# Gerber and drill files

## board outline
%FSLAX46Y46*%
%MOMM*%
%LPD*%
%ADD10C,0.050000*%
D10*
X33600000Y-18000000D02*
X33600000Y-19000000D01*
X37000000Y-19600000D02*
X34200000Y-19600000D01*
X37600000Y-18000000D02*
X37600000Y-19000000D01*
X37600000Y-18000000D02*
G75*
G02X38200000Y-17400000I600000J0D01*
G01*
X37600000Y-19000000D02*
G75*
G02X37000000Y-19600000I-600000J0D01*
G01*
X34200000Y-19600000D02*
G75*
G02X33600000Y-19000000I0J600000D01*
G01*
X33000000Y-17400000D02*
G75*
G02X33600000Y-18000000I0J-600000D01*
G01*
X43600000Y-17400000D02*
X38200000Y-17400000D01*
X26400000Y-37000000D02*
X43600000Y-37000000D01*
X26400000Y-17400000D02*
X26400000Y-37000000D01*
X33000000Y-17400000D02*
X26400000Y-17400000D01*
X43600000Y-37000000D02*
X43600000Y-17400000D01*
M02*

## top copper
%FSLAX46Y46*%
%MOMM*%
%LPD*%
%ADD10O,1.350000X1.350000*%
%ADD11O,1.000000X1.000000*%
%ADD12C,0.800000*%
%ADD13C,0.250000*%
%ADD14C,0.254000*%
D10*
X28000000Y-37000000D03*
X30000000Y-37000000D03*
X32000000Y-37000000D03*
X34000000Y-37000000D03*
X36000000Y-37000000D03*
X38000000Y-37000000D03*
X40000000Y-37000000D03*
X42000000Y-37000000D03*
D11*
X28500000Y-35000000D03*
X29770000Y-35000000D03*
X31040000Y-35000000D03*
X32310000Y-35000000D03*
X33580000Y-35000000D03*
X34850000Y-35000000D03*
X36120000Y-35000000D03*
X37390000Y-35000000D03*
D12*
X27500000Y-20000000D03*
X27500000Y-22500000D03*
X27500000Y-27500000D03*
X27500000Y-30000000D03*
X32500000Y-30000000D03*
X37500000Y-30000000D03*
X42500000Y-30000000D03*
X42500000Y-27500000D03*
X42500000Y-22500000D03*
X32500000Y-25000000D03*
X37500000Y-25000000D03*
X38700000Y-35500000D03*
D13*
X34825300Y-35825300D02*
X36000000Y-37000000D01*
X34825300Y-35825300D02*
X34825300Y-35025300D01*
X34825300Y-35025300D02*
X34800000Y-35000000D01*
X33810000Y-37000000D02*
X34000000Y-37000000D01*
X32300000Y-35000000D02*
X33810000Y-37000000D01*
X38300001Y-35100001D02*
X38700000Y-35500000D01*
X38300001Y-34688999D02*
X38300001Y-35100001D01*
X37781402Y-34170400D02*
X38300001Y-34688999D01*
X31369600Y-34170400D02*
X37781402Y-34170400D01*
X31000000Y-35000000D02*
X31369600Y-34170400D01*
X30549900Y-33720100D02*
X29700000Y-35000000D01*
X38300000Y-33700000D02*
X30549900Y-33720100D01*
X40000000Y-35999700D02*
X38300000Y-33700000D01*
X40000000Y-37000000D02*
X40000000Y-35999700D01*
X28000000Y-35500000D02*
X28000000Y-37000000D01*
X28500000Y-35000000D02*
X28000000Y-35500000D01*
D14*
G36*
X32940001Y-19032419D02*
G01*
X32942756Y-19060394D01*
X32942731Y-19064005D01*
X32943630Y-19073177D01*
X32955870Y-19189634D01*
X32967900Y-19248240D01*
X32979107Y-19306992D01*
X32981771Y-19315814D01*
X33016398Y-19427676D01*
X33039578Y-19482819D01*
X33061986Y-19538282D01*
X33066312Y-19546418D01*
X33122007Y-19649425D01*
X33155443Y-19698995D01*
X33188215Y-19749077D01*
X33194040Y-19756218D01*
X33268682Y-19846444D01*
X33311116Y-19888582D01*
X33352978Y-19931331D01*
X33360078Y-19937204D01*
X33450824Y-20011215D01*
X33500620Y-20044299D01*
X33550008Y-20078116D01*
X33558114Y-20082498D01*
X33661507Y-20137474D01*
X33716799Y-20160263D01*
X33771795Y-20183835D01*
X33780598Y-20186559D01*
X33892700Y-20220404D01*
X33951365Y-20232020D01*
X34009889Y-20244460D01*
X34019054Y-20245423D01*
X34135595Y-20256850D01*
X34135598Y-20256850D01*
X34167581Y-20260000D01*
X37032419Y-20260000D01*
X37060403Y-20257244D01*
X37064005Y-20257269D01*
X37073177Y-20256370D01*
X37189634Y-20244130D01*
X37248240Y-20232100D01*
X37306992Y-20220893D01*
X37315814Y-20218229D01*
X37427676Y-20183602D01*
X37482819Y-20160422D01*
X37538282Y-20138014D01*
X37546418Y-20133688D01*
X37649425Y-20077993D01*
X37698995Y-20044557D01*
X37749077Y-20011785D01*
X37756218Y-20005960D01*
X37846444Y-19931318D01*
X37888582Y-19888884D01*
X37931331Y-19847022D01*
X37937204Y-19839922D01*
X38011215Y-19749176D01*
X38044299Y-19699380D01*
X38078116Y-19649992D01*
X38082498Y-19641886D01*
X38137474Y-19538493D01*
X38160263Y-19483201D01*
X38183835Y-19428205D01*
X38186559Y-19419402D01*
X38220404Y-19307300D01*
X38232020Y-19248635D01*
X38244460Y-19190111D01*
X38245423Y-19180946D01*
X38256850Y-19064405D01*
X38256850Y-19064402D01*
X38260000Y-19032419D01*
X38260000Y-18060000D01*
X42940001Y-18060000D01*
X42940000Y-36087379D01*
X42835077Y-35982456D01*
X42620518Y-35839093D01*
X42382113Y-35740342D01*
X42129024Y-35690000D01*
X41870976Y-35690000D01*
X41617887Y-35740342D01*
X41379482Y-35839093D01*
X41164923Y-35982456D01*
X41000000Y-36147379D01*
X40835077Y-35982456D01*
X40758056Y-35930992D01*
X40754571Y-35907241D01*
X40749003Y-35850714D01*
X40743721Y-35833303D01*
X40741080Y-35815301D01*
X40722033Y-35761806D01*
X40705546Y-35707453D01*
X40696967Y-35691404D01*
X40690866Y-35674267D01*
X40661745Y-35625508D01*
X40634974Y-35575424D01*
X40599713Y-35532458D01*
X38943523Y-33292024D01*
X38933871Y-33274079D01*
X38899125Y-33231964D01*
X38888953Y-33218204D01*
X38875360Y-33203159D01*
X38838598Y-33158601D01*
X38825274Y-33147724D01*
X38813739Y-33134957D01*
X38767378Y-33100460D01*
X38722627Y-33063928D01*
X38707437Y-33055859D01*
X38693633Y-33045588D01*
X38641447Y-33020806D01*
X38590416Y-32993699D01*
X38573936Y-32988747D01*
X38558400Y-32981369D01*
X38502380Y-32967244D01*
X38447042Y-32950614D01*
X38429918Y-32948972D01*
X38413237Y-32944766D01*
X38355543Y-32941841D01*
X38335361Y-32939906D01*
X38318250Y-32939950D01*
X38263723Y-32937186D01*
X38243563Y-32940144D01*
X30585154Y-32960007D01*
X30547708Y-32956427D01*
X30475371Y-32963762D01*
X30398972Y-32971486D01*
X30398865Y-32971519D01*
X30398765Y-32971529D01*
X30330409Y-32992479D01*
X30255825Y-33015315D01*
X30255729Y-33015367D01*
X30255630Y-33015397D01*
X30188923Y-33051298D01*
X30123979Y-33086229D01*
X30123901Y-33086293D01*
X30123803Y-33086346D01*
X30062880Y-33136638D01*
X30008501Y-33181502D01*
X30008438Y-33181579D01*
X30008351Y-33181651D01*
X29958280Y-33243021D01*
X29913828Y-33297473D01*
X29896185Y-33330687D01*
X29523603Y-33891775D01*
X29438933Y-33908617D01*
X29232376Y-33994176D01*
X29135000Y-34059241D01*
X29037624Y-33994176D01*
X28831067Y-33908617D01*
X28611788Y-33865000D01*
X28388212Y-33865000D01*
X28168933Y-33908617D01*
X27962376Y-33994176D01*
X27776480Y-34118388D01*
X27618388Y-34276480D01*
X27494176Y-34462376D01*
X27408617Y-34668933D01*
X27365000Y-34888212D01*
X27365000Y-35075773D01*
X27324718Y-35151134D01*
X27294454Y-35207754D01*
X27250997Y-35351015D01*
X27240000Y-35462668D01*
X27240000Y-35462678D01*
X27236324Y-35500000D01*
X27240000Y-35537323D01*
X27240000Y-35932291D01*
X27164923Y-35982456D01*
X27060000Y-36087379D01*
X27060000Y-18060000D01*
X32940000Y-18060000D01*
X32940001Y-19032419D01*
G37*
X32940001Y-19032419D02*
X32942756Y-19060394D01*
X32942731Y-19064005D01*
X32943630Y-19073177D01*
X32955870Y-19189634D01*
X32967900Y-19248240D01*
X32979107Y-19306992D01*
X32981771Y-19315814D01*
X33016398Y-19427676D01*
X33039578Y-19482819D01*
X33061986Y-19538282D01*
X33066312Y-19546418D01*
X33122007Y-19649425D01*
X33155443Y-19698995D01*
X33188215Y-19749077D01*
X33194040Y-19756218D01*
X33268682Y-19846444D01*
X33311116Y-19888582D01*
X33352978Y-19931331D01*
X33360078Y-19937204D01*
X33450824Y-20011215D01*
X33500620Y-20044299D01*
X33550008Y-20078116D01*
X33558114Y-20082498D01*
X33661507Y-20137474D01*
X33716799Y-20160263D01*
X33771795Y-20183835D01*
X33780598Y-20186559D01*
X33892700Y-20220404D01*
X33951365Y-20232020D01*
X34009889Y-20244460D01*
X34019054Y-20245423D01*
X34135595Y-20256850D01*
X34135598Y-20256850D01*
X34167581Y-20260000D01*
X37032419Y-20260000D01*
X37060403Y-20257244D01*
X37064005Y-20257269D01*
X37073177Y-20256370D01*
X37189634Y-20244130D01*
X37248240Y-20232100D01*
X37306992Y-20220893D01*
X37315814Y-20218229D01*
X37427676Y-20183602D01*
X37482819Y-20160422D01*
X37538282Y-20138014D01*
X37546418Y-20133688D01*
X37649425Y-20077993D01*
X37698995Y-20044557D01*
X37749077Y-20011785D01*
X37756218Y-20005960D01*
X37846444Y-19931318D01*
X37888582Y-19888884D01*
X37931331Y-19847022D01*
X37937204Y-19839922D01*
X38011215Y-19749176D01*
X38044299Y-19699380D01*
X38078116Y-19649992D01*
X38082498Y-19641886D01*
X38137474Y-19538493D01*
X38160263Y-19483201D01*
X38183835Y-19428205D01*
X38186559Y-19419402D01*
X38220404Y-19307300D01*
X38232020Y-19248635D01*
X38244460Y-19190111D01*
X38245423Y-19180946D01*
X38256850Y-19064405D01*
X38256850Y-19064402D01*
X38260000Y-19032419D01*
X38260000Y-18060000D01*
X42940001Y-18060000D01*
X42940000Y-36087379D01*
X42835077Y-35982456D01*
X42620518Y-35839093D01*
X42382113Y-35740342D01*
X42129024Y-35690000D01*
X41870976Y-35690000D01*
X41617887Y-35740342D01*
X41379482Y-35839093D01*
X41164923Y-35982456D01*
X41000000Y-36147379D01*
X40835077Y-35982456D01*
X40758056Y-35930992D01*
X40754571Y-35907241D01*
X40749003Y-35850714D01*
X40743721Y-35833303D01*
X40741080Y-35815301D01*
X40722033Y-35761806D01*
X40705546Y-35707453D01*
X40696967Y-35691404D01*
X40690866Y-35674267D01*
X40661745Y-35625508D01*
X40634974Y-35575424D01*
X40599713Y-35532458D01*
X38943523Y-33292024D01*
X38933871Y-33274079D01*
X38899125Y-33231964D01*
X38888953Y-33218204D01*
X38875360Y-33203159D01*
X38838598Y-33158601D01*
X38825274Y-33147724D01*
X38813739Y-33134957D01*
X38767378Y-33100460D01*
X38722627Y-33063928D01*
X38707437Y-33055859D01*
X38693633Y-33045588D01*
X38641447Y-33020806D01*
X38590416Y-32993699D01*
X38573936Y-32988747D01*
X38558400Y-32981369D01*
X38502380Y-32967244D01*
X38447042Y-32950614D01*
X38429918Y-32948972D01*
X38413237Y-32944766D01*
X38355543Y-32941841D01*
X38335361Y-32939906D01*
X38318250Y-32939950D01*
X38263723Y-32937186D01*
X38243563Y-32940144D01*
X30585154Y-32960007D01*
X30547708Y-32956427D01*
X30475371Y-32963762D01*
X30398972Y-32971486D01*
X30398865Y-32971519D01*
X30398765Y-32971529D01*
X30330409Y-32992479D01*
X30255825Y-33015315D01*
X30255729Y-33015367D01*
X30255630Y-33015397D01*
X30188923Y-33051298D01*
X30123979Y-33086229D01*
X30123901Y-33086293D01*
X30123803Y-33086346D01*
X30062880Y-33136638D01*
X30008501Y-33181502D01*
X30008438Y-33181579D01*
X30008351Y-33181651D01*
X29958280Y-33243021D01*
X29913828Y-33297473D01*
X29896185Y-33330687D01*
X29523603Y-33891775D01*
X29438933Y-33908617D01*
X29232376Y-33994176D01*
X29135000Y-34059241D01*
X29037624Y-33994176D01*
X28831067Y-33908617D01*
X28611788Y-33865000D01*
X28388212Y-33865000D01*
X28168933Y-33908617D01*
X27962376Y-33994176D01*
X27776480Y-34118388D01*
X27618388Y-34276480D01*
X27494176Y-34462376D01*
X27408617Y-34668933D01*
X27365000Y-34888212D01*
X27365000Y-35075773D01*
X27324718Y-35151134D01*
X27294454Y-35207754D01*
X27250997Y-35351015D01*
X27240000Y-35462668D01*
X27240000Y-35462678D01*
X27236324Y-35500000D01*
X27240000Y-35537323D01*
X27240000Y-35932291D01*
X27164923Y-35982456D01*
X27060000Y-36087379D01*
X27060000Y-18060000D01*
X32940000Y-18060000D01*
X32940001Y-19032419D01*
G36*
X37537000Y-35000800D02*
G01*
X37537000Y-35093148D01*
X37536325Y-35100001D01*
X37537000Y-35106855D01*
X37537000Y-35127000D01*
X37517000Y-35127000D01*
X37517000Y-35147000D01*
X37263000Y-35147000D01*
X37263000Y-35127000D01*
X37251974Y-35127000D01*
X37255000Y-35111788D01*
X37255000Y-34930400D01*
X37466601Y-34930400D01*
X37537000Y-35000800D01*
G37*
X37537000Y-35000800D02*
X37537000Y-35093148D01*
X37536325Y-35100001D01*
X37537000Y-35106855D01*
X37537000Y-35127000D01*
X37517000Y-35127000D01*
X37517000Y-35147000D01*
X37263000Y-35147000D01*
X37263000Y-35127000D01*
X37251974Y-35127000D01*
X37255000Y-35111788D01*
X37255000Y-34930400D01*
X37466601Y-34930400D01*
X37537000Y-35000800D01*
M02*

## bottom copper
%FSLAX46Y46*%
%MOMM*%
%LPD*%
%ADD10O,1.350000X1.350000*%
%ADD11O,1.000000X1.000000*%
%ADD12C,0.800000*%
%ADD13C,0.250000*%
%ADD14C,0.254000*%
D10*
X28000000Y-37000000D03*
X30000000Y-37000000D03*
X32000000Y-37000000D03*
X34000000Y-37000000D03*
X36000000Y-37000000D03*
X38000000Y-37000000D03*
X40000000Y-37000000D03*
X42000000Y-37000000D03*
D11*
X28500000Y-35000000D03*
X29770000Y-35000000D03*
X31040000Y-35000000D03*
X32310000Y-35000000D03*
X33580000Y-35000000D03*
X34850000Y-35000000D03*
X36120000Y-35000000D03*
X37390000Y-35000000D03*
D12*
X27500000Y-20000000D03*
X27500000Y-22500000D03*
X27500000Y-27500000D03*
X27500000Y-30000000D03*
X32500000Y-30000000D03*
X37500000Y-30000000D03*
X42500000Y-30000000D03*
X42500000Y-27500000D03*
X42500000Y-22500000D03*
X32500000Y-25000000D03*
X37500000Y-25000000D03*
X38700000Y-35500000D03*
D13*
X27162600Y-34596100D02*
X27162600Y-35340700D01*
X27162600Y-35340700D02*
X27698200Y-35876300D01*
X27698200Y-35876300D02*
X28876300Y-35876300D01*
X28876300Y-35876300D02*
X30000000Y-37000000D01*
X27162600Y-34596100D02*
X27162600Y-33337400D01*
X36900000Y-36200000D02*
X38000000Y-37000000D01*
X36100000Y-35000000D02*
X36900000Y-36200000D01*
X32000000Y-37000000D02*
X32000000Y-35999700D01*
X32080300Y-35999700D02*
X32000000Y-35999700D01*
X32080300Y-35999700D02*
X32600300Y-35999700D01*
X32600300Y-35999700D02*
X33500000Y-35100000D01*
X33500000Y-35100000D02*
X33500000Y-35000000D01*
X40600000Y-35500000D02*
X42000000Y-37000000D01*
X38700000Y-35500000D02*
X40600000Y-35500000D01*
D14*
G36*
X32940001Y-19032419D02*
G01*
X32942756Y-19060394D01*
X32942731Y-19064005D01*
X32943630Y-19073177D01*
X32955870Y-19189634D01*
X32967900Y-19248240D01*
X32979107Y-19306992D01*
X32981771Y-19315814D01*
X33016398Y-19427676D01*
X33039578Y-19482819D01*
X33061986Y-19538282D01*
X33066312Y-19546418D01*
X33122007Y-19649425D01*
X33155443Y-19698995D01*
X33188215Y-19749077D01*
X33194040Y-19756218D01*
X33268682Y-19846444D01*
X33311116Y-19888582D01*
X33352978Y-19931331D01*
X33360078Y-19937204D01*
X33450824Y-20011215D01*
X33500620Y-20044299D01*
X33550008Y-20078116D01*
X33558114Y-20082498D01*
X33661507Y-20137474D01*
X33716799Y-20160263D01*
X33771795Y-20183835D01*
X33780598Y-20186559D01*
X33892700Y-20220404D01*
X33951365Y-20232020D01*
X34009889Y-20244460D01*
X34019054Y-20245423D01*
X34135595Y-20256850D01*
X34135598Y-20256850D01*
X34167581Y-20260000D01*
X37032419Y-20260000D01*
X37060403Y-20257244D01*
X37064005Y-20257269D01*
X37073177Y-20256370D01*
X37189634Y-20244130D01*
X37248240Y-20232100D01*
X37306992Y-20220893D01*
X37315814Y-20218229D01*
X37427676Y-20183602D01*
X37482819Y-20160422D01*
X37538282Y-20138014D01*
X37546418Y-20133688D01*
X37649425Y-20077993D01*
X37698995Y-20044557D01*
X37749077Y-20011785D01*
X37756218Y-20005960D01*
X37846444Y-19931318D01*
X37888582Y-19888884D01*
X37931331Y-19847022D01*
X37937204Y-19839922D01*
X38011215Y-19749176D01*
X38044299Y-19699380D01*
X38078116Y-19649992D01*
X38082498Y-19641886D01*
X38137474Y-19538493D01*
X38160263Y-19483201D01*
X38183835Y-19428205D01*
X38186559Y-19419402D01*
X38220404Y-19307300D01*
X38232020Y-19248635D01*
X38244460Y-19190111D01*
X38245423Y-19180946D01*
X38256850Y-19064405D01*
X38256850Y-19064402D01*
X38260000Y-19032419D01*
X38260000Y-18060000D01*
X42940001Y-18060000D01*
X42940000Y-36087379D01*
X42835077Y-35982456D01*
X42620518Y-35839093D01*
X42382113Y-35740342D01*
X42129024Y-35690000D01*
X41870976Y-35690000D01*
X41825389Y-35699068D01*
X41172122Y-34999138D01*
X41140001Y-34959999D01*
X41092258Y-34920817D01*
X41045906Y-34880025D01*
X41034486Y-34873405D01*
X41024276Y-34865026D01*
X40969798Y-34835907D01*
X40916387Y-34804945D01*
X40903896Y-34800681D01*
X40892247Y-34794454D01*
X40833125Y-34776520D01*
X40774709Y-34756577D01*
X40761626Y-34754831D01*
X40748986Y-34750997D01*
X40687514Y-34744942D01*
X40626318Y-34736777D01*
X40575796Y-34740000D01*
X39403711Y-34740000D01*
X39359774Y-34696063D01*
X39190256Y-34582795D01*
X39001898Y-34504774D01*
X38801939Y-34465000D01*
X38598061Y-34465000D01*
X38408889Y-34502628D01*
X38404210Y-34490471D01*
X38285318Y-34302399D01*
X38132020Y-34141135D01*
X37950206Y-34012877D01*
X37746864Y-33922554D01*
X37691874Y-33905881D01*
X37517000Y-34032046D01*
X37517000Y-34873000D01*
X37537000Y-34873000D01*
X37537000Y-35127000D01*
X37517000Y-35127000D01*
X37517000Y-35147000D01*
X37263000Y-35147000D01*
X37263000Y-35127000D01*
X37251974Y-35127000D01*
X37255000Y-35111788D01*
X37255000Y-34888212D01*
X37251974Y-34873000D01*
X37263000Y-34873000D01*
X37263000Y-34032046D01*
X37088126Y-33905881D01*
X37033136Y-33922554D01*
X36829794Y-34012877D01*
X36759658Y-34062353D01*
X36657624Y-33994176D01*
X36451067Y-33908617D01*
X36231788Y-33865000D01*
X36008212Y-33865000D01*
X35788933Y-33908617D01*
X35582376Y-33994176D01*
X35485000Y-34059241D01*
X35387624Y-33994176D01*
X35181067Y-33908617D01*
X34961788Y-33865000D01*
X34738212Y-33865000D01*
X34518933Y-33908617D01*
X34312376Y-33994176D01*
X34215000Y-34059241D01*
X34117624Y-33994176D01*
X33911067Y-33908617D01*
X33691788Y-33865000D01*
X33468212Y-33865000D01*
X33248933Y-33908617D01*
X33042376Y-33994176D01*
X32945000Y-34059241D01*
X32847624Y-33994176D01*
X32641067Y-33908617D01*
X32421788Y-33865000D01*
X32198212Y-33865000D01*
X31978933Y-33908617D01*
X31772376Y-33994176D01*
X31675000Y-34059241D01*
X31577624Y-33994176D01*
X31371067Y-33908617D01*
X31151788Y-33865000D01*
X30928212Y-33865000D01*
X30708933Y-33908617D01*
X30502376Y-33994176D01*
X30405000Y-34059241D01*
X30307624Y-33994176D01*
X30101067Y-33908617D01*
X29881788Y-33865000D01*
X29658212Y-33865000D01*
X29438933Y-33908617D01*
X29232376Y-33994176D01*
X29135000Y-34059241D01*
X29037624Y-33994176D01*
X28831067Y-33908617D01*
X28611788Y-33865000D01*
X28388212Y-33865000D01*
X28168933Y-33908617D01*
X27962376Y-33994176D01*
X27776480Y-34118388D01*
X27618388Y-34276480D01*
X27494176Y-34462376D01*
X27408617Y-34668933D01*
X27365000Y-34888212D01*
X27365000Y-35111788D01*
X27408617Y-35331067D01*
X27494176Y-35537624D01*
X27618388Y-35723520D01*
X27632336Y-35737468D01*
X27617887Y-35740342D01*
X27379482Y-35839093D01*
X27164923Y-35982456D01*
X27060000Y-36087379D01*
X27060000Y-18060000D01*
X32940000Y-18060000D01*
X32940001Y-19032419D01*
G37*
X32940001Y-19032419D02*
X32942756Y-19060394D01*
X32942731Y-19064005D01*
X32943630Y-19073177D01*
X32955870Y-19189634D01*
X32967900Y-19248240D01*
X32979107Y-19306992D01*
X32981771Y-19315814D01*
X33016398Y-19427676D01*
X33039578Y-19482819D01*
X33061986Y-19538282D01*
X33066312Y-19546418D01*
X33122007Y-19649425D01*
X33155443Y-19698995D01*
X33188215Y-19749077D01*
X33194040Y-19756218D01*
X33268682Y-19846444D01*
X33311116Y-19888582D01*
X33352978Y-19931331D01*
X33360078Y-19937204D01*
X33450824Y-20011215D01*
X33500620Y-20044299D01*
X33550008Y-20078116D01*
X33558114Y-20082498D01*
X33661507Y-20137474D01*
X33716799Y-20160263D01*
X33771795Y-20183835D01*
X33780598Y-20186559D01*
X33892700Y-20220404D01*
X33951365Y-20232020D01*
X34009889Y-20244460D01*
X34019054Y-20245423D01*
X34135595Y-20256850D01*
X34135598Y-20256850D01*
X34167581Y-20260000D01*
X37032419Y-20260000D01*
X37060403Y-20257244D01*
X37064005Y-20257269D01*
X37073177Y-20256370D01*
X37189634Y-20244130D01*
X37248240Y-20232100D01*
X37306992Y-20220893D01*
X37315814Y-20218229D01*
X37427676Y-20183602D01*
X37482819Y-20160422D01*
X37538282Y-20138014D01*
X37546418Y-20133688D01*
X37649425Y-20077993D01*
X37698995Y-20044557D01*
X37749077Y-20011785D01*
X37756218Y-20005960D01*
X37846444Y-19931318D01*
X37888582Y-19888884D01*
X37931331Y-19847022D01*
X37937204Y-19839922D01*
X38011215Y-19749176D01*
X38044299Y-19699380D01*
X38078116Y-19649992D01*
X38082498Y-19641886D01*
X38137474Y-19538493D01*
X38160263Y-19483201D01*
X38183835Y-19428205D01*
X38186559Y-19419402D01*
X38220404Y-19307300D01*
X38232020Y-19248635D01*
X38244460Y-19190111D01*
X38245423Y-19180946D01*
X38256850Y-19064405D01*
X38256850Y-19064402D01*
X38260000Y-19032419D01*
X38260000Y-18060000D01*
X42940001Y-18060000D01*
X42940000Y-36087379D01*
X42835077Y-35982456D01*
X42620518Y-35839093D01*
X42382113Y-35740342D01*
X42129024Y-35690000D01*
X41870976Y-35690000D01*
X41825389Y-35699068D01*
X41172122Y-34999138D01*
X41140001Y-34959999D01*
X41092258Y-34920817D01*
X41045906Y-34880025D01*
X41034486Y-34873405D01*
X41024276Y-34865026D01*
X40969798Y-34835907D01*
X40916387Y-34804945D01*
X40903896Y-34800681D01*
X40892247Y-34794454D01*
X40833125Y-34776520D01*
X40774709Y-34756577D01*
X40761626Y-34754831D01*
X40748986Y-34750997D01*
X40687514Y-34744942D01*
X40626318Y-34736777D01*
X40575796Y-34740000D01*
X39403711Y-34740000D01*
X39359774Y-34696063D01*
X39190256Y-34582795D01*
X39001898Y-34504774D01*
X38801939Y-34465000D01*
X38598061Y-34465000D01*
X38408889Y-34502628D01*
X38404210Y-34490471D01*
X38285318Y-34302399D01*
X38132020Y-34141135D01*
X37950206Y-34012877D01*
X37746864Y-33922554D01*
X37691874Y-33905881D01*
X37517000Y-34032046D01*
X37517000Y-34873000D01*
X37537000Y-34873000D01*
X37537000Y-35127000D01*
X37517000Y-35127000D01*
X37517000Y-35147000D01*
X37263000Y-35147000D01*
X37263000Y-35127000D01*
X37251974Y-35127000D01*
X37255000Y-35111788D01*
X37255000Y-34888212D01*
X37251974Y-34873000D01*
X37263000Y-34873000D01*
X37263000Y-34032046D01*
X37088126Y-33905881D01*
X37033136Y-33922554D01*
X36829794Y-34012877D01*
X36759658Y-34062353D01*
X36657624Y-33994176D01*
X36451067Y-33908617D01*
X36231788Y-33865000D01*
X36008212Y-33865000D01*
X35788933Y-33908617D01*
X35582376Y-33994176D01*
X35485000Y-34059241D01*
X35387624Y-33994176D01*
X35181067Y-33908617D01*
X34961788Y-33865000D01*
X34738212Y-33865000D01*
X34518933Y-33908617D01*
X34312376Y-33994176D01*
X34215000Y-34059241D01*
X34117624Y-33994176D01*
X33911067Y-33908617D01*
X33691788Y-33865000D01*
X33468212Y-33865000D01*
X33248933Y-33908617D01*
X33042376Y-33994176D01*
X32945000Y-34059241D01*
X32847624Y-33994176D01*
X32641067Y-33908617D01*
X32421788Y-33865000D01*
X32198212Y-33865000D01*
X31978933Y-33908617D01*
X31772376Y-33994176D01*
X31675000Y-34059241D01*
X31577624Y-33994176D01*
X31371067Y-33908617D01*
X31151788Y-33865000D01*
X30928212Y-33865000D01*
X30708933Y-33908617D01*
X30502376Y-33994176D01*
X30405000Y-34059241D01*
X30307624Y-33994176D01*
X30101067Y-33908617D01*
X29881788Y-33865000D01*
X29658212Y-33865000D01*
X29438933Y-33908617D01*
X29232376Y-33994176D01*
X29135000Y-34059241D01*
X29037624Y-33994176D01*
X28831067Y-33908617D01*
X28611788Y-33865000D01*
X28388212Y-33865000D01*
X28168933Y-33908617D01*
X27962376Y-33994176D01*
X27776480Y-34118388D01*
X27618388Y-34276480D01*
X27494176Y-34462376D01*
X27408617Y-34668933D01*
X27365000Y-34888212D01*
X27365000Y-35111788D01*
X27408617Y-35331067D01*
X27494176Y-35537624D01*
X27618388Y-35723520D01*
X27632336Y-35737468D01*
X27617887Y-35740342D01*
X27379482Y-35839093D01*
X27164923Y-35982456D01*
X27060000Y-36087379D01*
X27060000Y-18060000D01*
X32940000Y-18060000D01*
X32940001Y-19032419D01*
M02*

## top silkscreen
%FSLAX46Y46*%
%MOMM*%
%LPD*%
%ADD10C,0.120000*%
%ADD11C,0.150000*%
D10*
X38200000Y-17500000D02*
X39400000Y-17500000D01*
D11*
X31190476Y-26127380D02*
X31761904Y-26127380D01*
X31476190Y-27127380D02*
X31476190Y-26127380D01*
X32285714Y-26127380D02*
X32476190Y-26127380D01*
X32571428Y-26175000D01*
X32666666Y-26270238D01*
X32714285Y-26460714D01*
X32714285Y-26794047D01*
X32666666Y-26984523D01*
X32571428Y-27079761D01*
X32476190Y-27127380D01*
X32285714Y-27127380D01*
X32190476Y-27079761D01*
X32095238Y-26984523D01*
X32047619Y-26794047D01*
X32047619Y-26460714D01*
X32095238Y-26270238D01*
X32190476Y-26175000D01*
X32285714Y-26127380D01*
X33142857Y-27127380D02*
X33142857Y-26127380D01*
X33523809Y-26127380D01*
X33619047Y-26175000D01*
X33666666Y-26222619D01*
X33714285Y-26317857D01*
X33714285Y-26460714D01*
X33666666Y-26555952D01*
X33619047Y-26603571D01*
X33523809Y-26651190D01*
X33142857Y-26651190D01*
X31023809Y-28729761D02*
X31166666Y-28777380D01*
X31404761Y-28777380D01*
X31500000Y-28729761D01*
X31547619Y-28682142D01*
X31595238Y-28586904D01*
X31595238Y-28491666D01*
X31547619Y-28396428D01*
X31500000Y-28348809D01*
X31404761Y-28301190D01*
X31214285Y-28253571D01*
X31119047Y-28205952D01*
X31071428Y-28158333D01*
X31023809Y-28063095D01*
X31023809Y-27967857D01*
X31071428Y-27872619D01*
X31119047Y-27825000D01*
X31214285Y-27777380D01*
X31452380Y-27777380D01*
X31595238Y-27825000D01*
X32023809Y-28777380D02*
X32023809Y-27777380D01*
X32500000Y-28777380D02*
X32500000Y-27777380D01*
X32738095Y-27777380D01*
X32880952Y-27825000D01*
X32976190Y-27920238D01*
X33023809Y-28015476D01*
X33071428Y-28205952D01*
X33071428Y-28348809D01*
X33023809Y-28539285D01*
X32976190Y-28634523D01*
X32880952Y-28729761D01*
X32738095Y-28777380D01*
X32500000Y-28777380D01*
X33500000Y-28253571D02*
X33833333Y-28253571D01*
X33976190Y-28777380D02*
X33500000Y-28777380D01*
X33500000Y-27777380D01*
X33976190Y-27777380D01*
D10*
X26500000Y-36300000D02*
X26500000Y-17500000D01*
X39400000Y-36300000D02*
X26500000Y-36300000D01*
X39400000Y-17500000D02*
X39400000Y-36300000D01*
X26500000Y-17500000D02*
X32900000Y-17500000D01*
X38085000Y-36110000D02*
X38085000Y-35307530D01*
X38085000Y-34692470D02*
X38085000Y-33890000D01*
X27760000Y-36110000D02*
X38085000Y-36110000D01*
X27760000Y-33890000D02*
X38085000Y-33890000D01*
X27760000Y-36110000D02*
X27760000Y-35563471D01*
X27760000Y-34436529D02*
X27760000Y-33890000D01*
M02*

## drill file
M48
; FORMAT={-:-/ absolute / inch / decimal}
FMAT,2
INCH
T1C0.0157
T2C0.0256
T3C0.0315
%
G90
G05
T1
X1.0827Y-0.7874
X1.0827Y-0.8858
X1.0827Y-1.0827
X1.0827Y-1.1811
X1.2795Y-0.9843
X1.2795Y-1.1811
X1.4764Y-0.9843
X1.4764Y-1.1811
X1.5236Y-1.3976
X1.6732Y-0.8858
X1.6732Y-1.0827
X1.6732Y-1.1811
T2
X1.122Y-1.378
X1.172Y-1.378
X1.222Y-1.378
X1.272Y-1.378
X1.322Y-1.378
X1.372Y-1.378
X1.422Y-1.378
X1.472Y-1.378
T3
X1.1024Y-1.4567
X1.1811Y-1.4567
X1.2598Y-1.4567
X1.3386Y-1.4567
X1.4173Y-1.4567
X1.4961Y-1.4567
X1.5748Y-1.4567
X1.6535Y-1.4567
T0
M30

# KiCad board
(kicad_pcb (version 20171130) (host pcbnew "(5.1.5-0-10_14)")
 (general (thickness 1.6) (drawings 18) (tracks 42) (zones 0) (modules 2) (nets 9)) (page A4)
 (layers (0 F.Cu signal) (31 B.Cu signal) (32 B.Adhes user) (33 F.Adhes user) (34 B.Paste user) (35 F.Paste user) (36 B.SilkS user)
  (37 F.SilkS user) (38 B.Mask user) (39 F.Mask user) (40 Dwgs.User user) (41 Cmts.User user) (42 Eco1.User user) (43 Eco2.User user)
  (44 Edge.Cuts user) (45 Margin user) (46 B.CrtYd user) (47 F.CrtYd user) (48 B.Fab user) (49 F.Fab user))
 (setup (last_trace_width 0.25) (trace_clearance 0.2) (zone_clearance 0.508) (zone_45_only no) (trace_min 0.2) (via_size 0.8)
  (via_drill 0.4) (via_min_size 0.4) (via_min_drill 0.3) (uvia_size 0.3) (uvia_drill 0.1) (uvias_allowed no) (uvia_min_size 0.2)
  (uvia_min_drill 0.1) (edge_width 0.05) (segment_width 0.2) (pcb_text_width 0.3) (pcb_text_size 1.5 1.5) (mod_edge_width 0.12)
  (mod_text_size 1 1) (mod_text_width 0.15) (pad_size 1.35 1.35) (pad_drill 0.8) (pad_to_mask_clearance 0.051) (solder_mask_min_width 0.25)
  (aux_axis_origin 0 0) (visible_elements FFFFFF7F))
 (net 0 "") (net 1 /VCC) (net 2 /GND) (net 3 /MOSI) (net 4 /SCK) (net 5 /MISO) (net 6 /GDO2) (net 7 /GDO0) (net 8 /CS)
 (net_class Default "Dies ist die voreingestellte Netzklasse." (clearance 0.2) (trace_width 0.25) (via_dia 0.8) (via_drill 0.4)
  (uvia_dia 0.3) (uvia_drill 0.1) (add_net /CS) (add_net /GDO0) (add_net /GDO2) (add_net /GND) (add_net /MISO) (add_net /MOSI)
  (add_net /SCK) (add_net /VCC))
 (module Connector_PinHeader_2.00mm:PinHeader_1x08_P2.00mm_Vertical (layer B.Cu) (at 28 37 270)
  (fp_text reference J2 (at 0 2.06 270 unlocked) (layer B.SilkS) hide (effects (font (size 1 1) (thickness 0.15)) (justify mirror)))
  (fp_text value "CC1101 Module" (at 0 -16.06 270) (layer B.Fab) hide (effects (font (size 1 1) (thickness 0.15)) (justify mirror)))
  (pad 1 thru_hole oval (at 0 0 270) (size 1.35 1.35) (drill 0.8) (layers *.Cu *.Mask) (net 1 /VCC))
  (pad 2 thru_hole oval (at 0 -2 270) (size 1.35 1.35) (drill 0.8) (layers *.Cu *.Mask) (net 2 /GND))
  (pad 3 thru_hole oval (at 0 -4 270) (size 1.35 1.35) (drill 0.8) (layers *.Cu *.Mask) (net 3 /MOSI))
  (pad 4 thru_hole oval (at 0 -6 270) (size 1.35 1.35) (drill 0.8) (layers *.Cu *.Mask) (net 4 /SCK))
  (pad 5 thru_hole oval (at 0 -8 270) (size 1.35 1.35) (drill 0.8) (layers *.Cu *.Mask) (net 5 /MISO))
  (pad 6 thru_hole oval (at 0 -10 270) (size 1.35 1.35) (drill 0.8) (layers *.Cu *.Mask) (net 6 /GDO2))
  (pad 7 thru_hole oval (at 0 -12 270) (size 1.35 1.35) (drill 0.8) (layers *.Cu *.Mask) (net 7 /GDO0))
  (pad 8 thru_hole oval (at 0 -14 270) (size 1.35 1.35) (drill 0.8) (layers *.Cu *.Mask) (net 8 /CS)))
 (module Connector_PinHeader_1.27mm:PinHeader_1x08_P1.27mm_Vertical (layer F.Cu) (at 28.5 35 90)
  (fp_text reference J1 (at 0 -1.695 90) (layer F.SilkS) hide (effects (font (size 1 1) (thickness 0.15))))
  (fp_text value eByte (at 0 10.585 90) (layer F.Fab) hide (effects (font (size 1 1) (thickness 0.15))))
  (fp_line (start -1.11 9.585) (end -0.30753 9.585) (layer F.SilkS) (width 0.12))
  (fp_line (start 0.30753 9.585) (end 1.11 9.585) (layer F.SilkS) (width 0.12))
  (fp_line (start -1.11 -0.74) (end -1.11 9.585) (layer F.SilkS) (width 0.12))
  (fp_line (start 1.11 -0.74) (end 1.11 9.585) (layer F.SilkS) (width 0.12))
  (fp_line (start -1.11 -0.74) (end -0.563471 -0.74) (layer F.SilkS) (width 0.12))
  (fp_line (start 0.563471 -0.74) (end 1.11 -0.74) (layer F.SilkS) (width 0.12))
  (pad 1 thru_hole oval (at 0 0 90) (size 1 1) (drill 0.65) (layers *.Cu *.Mask) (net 1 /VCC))
  (pad 2 thru_hole oval (at 0 1.27 90) (size 1 1) (drill 0.65) (layers *.Cu *.Mask) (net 7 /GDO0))
  (pad 3 thru_hole oval (at 0 2.54 90) (size 1 1) (drill 0.65) (layers *.Cu *.Mask) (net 8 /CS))
  (pad 4 thru_hole oval (at 0 3.81 90) (size 1 1) (drill 0.65) (layers *.Cu *.Mask) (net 4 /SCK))
  (pad 5 thru_hole oval (at 0 5.08 90) (size 1 1) (drill 0.65) (layers *.Cu *.Mask) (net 3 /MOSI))
  (pad 6 thru_hole oval (at 0 6.35 90) (size 1 1) (drill 0.65) (layers *.Cu *.Mask) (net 5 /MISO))
  (pad 7 thru_hole oval (at 0 7.62 90) (size 1 1) (drill 0.65) (layers *.Cu *.Mask) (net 6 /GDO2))
  (pad 8 thru_hole oval (at 0 8.89 90) (size 1 1) (drill 0.65) (layers *.Cu *.Mask) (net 2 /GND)))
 (gr_line (start 38.2 17.5) (end 39.4 17.5) (layer F.SilkS) (width 0.12))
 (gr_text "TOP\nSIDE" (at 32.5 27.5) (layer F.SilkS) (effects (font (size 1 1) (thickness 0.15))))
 (gr_line (start 26.5 36.3) (end 26.5 17.5) (layer F.SilkS) (width 0.12))
 (gr_line (start 39.4 36.3) (end 26.5 36.3) (layer F.SilkS) (width 0.12))
 (gr_line (start 39.4 17.5) (end 39.4 36.3) (layer F.SilkS) (width 0.12))
 (gr_line (start 26.5 17.5) (end 32.9 17.5) (layer F.SilkS) (width 0.12))
 (gr_line (start 33.6 18) (end 33.6 19) (layer Edge.Cuts) (width 0.05))
 (gr_line (start 37 19.6) (end 34.2 19.6) (layer Edge.Cuts) (width 0.05))
 (gr_line (start 37.6 18) (end 37.6 19) (layer Edge.Cuts) (width 0.05))
 (gr_arc (start 38.2 18) (end 38.2 17.4) (angle -90) (layer Edge.Cuts) (width 0.05))
 (gr_arc (start 37 19) (end 37 19.6) (angle -90) (layer Edge.Cuts) (width 0.05))
 (gr_arc (start 34.2 19) (end 33.6 19) (angle -90) (layer Edge.Cuts) (width 0.05))
 (gr_arc (start 33 18) (end 33.6 18) (angle -90) (layer Edge.Cuts) (width 0.05))
 (gr_line (start 43.6 17.4) (end 38.2 17.4) (layer Edge.Cuts) (width 0.05))
 (gr_line (start 26.4 37) (end 43.6 37) (layer Edge.Cuts) (width 0.05))
 (gr_line (start 26.4 17.4) (end 26.4 37) (layer Edge.Cuts) (width 0.05))
 (gr_line (start 33 17.4) (end 26.4 17.4) (layer Edge.Cuts) (width 0.05))
 (gr_line (start 43.6 37) (end 43.6 17.4) (layer Edge.Cuts) (width 0.05))
 (segment (start 27.1626 34.5961) (end 27.1626 35.3407) (width 0.25) (layer B.Cu) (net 2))
 (segment (start 27.1626 35.3407) (end 27.6982 35.8763) (width 0.25) (layer B.Cu) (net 2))
 (segment (start 27.6982 35.8763) (end 28.8763 35.8763) (width 0.25) (layer B.Cu) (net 2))
 (segment (start 28.8763 35.8763) (end 30 37) (width 0.25) (layer B.Cu) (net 2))
 (segment (start 27.1626 34.5961) (end 27.1626 33.3374) (width 0.25) (layer B.Cu) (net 2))
 (via (at 27.5 20) (size 0.8) (drill 0.4) (layers F.Cu B.Cu) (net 2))
 (via (at 27.5 22.5) (size 0.8) (drill 0.4) (layers F.Cu B.Cu) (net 2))
 (via (at 27.5 27.5) (size 0.8) (drill 0.4) (layers F.Cu B.Cu) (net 2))
 (via (at 27.5 30) (size 0.8) (drill 0.4) (layers F.Cu B.Cu) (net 2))
 (via (at 32.5 30) (size 0.8) (drill 0.4) (layers F.Cu B.Cu) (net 2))
 (via (at 37.5 30) (size 0.8) (drill 0.4) (layers F.Cu B.Cu) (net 2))
 (via (at 42.5 30) (size 0.8) (drill 0.4) (layers F.Cu B.Cu) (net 2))
 (via (at 42.5 27.5) (size 0.8) (drill 0.4) (layers F.Cu B.Cu) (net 2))
 (via (at 42.5 22.5) (size 0.8) (drill 0.4) (layers F.Cu B.Cu) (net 2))
 (via (at 32.5 25) (size 0.8) (drill 0.4) (layers F.Cu B.Cu) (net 2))
 (via (at 37.5 25) (size 0.8) (drill 0.4) (layers F.Cu B.Cu) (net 2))
 (segment (start 36.9 36.2) (end 38 37) (width 0.25) (layer B.Cu) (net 6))
 (segment (start 36.1 35) (end 36.9 36.2) (width 0.25) (layer B.Cu) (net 6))
 (segment (start 34.8253 35.8253) (end 36 37) (width 0.25) (layer F.Cu) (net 5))
 (segment (start 34.8253 35.8253) (end 34.8253 35.0253) (width 0.25) (layer F.Cu) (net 5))
 (segment (start 34.8253 35.0253) (end 34.8 35) (width 0.25) (layer F.Cu) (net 5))
 (segment (start 32 37) (end 32 35.9997) (width 0.25) (layer B.Cu) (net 3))
 (segment (start 32.0803 35.9997) (end 32 35.9997) (width 0.25) (layer B.Cu) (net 3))
 (segment (start 32.0803 35.9997) (end 32.6003 35.9997) (width 0.25) (layer B.Cu) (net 3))
 (segment (start 32.6003 35.9997) (end 33.5 35.1) (width 0.25) (layer B.Cu) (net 3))
 (segment (start 33.5 35.1) (end 33.5 35) (width 0.25) (layer B.Cu) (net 3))
 (segment (start 33.81 37) (end 34 37) (width 0.25) (layer F.Cu) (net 4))
 (segment (start 32.3 35) (end 33.81 37) (width 0.25) (layer F.Cu) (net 4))
 (segment (start 40.6 35.5) (end 42 37) (width 0.25) (layer B.Cu) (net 8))
 (segment (start 38.7 35.5) (end 40.6 35.5) (width 0.25) (layer B.Cu) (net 8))
 (segment (start 38.300001 35.100001) (end 38.7 35.5) (width 0.25) (layer F.Cu) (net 8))
 (via (at 38.7 35.5) (size 0.8) (drill 0.4) (layers F.Cu B.Cu) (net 8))
 (segment (start 38.300001 34.688999) (end 38.300001 35.100001) (width 0.25) (layer F.Cu) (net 8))
 (segment (start 37.781402 34.1704) (end 38.300001 34.688999) (width 0.25) (layer F.Cu) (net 8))
 (segment (start 31.3696 34.1704) (end 37.781402 34.1704) (width 0.25) (layer F.Cu) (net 8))
 (segment (start 31 35) (end 31.3696 34.1704) (width 0.25) (layer F.Cu) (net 8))
 (segment (start 30.5499 33.7201) (end 29.7 35) (width 0.25) (layer F.Cu) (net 7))
 (segment (start 38.3 33.7) (end 30.5499 33.7201) (width 0.25) (layer F.Cu) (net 7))
 (segment (start 40 35.9997) (end 38.3 33.7) (width 0.25) (layer F.Cu) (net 7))
 (segment (start 40 37) (end 40 35.9997) (width 0.25) (layer F.Cu) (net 7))
 (segment (start 28 35.5) (end 28 37) (width 0.25) (layer F.Cu) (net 1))
 (segment (start 28.5 35) (end 28 35.5) (width 0.25) (layer F.Cu) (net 1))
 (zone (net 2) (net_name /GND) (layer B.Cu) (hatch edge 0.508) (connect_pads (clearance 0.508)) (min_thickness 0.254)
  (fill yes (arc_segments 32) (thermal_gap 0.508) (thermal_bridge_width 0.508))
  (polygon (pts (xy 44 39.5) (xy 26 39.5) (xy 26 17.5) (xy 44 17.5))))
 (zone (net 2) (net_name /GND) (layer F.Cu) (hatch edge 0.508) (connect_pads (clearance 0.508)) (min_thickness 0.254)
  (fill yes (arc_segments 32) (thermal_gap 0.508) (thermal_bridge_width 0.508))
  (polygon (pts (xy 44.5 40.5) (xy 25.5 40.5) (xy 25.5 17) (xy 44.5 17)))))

